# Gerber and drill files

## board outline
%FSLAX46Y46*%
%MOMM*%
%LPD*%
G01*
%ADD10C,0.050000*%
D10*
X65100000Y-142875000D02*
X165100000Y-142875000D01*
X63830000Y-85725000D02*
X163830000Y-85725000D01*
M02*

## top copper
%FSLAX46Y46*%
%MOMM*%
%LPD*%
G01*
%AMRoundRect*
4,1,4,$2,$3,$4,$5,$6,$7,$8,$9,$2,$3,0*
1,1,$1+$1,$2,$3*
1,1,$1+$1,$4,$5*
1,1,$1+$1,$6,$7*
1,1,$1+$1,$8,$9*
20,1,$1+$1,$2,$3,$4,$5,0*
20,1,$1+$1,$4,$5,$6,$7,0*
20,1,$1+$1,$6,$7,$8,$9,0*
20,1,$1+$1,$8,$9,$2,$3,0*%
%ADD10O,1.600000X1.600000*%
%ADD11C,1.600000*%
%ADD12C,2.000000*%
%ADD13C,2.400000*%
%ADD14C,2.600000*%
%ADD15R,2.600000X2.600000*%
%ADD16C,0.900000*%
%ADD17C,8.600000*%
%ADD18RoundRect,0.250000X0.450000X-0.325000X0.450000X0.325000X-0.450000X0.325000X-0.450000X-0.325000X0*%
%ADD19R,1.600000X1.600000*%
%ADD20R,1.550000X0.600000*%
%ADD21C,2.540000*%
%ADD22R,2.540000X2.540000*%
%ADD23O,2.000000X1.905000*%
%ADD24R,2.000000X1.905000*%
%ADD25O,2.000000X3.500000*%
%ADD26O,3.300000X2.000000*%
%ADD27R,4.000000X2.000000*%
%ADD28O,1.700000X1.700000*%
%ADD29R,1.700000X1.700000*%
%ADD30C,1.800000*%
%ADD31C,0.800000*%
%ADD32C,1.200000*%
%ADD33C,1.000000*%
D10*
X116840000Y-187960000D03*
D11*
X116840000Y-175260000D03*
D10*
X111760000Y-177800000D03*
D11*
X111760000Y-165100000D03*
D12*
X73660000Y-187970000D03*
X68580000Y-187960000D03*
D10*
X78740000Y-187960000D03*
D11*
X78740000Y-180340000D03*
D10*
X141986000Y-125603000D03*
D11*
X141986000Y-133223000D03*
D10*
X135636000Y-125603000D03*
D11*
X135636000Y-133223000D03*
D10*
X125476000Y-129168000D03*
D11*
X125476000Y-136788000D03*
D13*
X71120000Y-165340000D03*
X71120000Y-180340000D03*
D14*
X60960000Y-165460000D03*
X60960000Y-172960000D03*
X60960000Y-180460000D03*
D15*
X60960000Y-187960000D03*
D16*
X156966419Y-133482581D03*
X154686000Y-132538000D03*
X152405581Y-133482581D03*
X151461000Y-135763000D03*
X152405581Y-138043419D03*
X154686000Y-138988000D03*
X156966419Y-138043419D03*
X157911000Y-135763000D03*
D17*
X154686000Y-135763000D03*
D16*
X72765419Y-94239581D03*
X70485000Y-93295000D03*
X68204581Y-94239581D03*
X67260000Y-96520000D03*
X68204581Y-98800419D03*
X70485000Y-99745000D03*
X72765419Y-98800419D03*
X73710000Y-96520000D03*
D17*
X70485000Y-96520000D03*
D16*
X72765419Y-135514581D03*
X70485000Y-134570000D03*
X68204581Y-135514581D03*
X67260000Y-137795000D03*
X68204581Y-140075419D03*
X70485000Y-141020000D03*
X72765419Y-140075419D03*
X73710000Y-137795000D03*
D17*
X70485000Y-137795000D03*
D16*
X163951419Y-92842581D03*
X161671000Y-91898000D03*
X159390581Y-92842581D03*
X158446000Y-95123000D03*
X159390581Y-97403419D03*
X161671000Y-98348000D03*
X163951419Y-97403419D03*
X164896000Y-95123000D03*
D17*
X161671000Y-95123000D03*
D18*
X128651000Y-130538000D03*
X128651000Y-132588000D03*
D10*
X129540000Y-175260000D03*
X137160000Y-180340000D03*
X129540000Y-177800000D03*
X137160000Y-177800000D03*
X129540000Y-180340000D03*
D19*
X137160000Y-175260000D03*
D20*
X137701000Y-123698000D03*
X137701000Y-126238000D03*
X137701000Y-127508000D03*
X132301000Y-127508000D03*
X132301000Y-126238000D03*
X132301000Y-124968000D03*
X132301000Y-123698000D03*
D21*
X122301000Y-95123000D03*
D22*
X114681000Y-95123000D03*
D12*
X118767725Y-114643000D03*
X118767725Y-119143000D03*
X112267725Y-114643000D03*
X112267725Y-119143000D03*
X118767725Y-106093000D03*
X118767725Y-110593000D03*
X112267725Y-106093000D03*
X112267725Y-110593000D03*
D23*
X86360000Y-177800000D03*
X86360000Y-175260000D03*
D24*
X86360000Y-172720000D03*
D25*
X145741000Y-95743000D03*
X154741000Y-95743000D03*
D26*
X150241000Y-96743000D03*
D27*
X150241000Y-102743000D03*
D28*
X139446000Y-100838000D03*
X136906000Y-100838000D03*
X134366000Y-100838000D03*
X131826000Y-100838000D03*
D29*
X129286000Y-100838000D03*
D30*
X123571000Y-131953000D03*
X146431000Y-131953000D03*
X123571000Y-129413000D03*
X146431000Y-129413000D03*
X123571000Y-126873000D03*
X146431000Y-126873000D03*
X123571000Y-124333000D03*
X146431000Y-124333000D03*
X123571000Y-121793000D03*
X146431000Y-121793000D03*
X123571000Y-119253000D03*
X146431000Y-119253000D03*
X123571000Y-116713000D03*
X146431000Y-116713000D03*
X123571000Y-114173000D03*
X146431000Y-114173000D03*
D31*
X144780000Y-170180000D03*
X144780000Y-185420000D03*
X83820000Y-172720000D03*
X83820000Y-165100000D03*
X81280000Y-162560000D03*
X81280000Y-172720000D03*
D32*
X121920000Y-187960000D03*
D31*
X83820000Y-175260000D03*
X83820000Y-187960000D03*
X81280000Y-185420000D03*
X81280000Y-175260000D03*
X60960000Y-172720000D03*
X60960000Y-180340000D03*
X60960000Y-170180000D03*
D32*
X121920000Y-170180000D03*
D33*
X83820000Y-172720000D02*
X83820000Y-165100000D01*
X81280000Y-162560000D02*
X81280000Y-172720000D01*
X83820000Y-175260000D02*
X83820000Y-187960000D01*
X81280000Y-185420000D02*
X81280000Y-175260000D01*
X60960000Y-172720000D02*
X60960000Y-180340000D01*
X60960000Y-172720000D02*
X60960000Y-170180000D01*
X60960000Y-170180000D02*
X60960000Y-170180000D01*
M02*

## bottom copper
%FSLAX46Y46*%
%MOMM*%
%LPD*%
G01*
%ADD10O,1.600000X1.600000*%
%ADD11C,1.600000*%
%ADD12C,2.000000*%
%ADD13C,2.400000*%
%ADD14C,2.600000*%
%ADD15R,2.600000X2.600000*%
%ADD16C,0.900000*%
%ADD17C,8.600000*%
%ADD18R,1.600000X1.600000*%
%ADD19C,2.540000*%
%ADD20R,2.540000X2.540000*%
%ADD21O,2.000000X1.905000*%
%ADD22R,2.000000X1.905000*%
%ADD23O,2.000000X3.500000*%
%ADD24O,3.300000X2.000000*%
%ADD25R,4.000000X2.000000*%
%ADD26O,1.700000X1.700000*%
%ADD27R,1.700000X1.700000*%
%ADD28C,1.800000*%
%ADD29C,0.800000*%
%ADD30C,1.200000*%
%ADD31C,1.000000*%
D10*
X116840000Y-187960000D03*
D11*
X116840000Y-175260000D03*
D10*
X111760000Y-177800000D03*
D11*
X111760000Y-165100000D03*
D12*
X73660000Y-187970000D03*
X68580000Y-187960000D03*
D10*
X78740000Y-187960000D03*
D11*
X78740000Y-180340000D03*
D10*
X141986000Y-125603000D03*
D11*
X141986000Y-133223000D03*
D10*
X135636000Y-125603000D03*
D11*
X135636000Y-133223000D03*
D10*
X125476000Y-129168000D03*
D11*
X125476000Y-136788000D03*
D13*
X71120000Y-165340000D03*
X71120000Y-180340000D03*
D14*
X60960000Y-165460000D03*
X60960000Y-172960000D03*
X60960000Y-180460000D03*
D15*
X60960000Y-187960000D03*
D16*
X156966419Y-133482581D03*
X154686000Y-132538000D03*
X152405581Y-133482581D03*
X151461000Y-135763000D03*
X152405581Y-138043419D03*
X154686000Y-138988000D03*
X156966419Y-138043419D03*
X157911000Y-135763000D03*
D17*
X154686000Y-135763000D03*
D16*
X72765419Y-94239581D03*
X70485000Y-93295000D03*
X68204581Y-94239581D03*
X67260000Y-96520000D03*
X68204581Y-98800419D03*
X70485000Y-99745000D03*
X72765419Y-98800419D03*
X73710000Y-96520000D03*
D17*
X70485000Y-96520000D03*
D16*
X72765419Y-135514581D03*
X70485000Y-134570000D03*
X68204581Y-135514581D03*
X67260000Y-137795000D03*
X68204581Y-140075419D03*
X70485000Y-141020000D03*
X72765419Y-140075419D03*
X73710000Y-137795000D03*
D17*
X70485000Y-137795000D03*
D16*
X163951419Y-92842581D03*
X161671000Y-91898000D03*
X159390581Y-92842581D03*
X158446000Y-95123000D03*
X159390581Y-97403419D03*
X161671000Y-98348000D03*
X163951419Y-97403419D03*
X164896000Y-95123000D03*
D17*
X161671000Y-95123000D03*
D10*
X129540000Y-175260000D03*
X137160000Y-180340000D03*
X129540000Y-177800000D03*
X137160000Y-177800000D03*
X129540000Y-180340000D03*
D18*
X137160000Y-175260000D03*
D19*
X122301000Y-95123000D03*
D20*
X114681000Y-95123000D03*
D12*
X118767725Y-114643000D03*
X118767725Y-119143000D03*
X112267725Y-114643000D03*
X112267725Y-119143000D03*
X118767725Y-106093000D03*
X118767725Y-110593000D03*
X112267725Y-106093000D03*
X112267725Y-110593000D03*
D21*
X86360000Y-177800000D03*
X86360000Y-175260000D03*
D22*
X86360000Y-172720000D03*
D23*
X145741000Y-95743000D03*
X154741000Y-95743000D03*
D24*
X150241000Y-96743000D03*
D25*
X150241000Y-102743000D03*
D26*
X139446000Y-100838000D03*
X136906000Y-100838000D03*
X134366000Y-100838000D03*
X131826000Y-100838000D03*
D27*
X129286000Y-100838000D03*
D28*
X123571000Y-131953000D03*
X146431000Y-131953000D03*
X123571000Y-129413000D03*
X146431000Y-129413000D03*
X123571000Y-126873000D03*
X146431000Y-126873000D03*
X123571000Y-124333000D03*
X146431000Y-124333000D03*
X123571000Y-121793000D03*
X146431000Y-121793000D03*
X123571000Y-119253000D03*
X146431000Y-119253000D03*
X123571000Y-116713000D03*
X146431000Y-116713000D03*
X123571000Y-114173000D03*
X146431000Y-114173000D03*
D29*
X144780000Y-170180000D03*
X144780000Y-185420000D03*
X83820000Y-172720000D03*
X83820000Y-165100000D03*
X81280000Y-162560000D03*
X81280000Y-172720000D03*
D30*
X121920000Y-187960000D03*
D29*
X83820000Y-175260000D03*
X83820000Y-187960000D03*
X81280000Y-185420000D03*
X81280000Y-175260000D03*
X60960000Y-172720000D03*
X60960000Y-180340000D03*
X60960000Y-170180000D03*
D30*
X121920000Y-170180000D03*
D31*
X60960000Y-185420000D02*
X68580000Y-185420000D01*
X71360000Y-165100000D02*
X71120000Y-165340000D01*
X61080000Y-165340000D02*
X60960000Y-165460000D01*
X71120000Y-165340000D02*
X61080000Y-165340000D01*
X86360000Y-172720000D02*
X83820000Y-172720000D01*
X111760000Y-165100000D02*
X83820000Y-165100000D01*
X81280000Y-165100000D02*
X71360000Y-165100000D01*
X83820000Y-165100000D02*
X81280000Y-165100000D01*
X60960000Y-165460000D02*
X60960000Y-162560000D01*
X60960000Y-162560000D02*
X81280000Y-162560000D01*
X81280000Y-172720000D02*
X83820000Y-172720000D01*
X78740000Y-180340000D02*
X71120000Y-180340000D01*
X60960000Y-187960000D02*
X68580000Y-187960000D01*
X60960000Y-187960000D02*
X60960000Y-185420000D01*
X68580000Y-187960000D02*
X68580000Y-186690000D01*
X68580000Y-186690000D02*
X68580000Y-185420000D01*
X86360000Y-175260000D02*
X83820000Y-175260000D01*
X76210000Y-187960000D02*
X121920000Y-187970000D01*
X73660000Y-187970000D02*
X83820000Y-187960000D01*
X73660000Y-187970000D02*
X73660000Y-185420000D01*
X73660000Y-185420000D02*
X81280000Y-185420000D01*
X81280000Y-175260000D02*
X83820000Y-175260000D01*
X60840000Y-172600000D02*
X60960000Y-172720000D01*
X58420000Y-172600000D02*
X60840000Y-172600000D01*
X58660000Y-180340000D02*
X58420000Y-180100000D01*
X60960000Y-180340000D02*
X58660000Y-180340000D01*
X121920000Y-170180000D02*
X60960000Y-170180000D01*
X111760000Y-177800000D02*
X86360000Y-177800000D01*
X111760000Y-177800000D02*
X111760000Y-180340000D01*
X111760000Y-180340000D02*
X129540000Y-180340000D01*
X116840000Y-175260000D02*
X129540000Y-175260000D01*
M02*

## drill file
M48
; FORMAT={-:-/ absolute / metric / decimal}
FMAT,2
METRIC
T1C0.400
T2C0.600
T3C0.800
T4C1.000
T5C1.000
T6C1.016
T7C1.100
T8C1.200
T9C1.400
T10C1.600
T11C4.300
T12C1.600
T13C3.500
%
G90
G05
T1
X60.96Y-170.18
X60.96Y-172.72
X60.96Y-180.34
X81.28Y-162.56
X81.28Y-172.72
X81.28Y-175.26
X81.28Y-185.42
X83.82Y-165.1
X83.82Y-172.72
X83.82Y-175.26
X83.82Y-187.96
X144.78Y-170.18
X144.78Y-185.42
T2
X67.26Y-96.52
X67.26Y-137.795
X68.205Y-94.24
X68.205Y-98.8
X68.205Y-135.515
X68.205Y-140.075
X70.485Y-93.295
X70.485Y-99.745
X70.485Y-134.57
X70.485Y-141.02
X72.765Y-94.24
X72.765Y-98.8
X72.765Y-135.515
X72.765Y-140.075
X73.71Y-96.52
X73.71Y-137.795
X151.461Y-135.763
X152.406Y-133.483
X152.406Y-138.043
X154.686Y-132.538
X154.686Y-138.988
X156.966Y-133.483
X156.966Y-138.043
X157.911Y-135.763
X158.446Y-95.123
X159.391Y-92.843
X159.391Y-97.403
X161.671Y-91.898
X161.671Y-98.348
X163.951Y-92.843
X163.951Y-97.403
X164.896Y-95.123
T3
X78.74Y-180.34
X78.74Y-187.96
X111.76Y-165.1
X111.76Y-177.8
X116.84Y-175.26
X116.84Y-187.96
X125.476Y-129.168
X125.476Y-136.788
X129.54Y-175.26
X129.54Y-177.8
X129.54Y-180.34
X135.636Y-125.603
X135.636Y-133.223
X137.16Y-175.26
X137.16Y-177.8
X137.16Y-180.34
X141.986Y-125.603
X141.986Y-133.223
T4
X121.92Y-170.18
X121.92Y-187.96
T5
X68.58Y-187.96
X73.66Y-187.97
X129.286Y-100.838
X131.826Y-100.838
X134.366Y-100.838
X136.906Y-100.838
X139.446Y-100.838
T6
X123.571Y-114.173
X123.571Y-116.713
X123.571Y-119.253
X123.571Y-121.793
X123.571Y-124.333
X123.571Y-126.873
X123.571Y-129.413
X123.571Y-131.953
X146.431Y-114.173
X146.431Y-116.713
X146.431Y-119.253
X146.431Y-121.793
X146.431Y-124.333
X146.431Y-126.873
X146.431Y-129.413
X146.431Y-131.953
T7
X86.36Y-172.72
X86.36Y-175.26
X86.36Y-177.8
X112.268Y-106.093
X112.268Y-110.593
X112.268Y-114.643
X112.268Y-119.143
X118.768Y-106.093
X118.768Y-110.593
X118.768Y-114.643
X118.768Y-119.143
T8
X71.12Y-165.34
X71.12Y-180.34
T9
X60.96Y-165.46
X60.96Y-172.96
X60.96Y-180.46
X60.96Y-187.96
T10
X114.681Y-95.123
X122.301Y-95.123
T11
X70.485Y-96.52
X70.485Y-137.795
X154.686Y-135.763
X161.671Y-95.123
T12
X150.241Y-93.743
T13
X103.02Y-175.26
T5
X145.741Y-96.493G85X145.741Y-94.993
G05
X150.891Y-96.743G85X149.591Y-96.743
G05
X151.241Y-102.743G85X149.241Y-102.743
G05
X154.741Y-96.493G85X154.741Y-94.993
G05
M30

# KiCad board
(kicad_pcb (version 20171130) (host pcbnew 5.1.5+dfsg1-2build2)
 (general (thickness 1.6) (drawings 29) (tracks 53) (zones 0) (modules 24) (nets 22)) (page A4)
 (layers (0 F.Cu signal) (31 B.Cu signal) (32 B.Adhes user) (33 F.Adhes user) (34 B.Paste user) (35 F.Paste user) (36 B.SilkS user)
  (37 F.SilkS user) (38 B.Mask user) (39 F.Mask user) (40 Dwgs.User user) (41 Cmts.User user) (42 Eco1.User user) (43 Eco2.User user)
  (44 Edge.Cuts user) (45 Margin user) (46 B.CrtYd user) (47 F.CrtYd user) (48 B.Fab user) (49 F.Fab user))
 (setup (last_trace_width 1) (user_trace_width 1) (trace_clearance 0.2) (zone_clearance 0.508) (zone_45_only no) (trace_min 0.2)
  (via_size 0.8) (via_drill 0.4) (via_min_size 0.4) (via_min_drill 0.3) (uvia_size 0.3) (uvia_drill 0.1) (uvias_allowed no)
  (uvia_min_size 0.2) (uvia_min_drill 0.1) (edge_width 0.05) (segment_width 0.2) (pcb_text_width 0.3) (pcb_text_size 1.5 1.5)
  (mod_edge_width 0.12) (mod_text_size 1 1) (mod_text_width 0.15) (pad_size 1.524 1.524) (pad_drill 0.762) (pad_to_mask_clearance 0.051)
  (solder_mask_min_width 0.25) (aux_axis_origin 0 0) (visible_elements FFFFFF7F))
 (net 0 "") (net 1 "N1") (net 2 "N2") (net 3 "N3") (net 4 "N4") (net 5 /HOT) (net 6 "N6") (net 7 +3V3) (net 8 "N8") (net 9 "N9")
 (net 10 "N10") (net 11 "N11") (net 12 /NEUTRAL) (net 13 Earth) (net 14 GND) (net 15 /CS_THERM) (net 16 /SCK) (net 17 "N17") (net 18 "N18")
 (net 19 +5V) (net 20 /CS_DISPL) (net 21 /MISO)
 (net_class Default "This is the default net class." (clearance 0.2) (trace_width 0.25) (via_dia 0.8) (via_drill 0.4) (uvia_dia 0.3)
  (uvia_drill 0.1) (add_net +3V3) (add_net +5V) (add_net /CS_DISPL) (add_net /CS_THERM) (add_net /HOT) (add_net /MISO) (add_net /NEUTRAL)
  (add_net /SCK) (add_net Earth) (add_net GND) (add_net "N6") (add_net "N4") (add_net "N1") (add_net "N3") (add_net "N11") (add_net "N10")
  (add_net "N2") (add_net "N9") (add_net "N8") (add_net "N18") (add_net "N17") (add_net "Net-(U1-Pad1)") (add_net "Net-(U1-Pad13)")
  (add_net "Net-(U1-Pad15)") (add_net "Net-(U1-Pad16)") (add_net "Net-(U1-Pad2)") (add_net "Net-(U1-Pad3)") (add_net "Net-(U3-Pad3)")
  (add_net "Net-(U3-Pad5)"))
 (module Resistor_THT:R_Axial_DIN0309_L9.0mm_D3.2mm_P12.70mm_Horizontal (layer F.Cu) (at 116.84 175.26 270)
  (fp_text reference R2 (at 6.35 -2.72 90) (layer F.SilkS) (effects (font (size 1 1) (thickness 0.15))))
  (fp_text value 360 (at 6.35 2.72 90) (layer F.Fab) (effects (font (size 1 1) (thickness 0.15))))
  (pad 2 thru_hole oval (at 12.7 0 270) (size 1.6 1.6) (drill 0.8) (layers *.Cu *.Mask) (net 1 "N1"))
  (pad 1 thru_hole circle (at 0 0 270) (size 1.6 1.6) (drill 0.8) (layers *.Cu *.Mask) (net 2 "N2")))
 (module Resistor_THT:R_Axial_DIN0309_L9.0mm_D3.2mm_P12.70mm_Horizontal (layer F.Cu) (at 111.76 165.1 270)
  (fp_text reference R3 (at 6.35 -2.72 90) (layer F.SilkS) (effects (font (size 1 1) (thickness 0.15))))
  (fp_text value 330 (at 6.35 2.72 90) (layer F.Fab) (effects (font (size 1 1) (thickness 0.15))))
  (pad 2 thru_hole oval (at 12.7 0 270) (size 1.6 1.6) (drill 0.8) (layers *.Cu *.Mask) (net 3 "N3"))
  (pad 1 thru_hole circle (at 0 0 270) (size 1.6 1.6) (drill 0.8) (layers *.Cu *.Mask) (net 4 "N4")))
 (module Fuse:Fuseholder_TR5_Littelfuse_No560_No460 (layer F.Cu) (at 68.58 187.96)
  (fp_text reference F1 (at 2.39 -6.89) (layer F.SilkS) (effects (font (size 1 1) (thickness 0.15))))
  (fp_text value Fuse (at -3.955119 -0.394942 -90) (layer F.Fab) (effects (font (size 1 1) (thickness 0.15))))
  (pad 2 thru_hole circle (at 5.08 0.01) (size 2 2) (drill 1) (layers *.Cu *.Mask) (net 1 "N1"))
  (pad 1 thru_hole circle (at 0 0) (size 2 2) (drill 1) (layers *.Cu *.Mask) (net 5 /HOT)))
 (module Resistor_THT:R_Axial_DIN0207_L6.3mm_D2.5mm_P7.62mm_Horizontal (layer F.Cu) (at 78.74 180.34 270)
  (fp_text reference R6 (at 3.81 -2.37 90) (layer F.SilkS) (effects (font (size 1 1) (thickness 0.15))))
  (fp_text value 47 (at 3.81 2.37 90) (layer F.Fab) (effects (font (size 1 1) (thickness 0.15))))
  (pad 2 thru_hole oval (at 7.62 0 270) (size 1.6 1.6) (drill 0.8) (layers *.Cu *.Mask) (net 1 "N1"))
  (pad 1 thru_hole circle (at 0 0 270) (size 1.6 1.6) (drill 0.8) (layers *.Cu *.Mask) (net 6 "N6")))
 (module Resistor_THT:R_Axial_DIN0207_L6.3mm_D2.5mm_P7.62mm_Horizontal (layer F.Cu) (at 141.986 133.223 90)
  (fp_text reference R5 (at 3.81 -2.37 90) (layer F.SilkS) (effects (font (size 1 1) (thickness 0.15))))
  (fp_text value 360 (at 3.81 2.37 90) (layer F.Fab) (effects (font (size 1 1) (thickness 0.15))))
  (pad 2 thru_hole oval (at 7.62 0 90) (size 1.6 1.6) (drill 0.8) (layers *.Cu *.Mask) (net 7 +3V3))
  (pad 1 thru_hole circle (at 0 0 90) (size 1.6 1.6) (drill 0.8) (layers *.Cu *.Mask) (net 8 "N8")))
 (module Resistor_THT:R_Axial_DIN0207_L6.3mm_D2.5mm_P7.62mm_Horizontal (layer F.Cu) (at 135.636 133.223 90)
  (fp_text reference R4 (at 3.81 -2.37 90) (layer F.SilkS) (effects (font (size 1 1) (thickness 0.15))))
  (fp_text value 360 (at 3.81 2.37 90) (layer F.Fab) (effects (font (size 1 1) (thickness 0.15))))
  (pad 2 thru_hole oval (at 7.62 0 90) (size 1.6 1.6) (drill 0.8) (layers *.Cu *.Mask) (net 7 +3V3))
  (pad 1 thru_hole circle (at 0 0 90) (size 1.6 1.6) (drill 0.8) (layers *.Cu *.Mask) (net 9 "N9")))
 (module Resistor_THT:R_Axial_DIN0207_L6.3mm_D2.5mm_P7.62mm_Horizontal (layer F.Cu) (at 125.476 136.788 90)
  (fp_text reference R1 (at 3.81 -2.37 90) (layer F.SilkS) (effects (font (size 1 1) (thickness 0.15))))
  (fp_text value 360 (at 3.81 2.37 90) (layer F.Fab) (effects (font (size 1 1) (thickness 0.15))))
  (pad 2 thru_hole oval (at 7.62 0 90) (size 1.6 1.6) (drill 0.8) (layers *.Cu *.Mask) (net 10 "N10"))
  (pad 1 thru_hole circle (at 0 0 90) (size 1.6 1.6) (drill 0.8) (layers *.Cu *.Mask) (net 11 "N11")))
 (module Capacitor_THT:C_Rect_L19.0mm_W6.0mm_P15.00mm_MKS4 (layer F.Cu) (at 71.12 180.34 90)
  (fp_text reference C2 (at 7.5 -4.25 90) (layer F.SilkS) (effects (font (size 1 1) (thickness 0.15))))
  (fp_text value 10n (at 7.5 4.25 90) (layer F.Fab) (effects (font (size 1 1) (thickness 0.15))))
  (pad 2 thru_hole circle (at 15 0 90) (size 2.4 2.4) (drill 1.2) (layers *.Cu *.Mask) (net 4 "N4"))
  (pad 1 thru_hole circle (at 0 0 90) (size 2.4 2.4) (drill 1.2) (layers *.Cu *.Mask) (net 6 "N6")))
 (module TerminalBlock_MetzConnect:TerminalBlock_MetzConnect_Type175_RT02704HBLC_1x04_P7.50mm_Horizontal (layer F.Cu) (at 60.96 187.96 90)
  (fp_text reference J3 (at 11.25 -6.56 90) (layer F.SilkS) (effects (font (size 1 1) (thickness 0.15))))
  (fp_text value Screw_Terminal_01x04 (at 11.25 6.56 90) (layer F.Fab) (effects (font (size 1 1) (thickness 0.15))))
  (pad 4 thru_hole circle (at 22.5 0 90) (size 2.6 2.6) (drill 1.4) (layers *.Cu *.Mask) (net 4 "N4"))
  (pad 3 thru_hole circle (at 15 0 90) (size 2.6 2.6) (drill 1.4) (layers *.Cu *.Mask) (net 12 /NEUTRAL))
  (pad 2 thru_hole circle (at 7.5 0 90) (size 2.6 2.6) (drill 1.4) (layers *.Cu *.Mask) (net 12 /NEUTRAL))
  (pad 1 thru_hole rect (at 0 0 90) (size 2.6 2.6) (drill 1.4) (layers *.Cu *.Mask) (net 5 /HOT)))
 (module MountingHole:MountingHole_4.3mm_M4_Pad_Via (layer F.Cu) (at 154.686 135.763)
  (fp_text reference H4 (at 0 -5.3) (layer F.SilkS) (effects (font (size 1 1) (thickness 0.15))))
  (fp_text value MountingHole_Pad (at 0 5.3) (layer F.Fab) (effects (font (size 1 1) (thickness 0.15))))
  (pad 1 thru_hole circle (at 2.280419 -2.280419) (size 0.9 0.9) (drill 0.6) (layers *.Cu *.Mask) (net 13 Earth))
  (pad 1 thru_hole circle (at 0 -3.225) (size 0.9 0.9) (drill 0.6) (layers *.Cu *.Mask) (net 13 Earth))
  (pad 1 thru_hole circle (at -2.280419 -2.280419) (size 0.9 0.9) (drill 0.6) (layers *.Cu *.Mask) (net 13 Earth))
  (pad 1 thru_hole circle (at -3.225 0) (size 0.9 0.9) (drill 0.6) (layers *.Cu *.Mask) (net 13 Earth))
  (pad 1 thru_hole circle (at -2.280419 2.280419) (size 0.9 0.9) (drill 0.6) (layers *.Cu *.Mask) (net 13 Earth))
  (pad 1 thru_hole circle (at 0 3.225) (size 0.9 0.9) (drill 0.6) (layers *.Cu *.Mask) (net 13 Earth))
  (pad 1 thru_hole circle (at 2.280419 2.280419) (size 0.9 0.9) (drill 0.6) (layers *.Cu *.Mask) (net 13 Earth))
  (pad 1 thru_hole circle (at 3.225 0) (size 0.9 0.9) (drill 0.6) (layers *.Cu *.Mask) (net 13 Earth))
  (pad 1 thru_hole circle (at 0 0) (size 8.6 8.6) (drill 4.3) (layers *.Cu *.Mask) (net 13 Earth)))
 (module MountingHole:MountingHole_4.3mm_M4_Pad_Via (layer F.Cu) (at 70.485 96.52)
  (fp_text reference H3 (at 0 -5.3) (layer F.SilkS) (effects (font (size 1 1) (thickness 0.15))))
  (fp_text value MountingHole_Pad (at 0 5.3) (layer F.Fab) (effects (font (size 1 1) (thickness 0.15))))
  (pad 1 thru_hole circle (at 2.280419 -2.280419) (size 0.9 0.9) (drill 0.6) (layers *.Cu *.Mask) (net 13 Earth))
  (pad 1 thru_hole circle (at 0 -3.225) (size 0.9 0.9) (drill 0.6) (layers *.Cu *.Mask) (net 13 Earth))
  (pad 1 thru_hole circle (at -2.280419 -2.280419) (size 0.9 0.9) (drill 0.6) (layers *.Cu *.Mask) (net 13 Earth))
  (pad 1 thru_hole circle (at -3.225 0) (size 0.9 0.9) (drill 0.6) (layers *.Cu *.Mask) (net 13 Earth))
  (pad 1 thru_hole circle (at -2.280419 2.280419) (size 0.9 0.9) (drill 0.6) (layers *.Cu *.Mask) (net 13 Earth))
  (pad 1 thru_hole circle (at 0 3.225) (size 0.9 0.9) (drill 0.6) (layers *.Cu *.Mask) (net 13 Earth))
  (pad 1 thru_hole circle (at 2.280419 2.280419) (size 0.9 0.9) (drill 0.6) (layers *.Cu *.Mask) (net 13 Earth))
  (pad 1 thru_hole circle (at 3.225 0) (size 0.9 0.9) (drill 0.6) (layers *.Cu *.Mask) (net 13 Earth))
  (pad 1 thru_hole circle (at 0 0) (size 8.6 8.6) (drill 4.3) (layers *.Cu *.Mask) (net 13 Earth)))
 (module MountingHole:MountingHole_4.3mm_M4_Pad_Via (layer F.Cu) (at 70.485 137.795)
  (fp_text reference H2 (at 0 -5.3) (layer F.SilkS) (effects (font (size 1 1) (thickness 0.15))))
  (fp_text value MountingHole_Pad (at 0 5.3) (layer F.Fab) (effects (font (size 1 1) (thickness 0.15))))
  (pad 1 thru_hole circle (at 2.280419 -2.280419) (size 0.9 0.9) (drill 0.6) (layers *.Cu *.Mask) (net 13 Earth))
  (pad 1 thru_hole circle (at 0 -3.225) (size 0.9 0.9) (drill 0.6) (layers *.Cu *.Mask) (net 13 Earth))
  (pad 1 thru_hole circle (at -2.280419 -2.280419) (size 0.9 0.9) (drill 0.6) (layers *.Cu *.Mask) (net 13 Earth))
  (pad 1 thru_hole circle (at -3.225 0) (size 0.9 0.9) (drill 0.6) (layers *.Cu *.Mask) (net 13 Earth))
  (pad 1 thru_hole circle (at -2.280419 2.280419) (size 0.9 0.9) (drill 0.6) (layers *.Cu *.Mask) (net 13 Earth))
  (pad 1 thru_hole circle (at 0 3.225) (size 0.9 0.9) (drill 0.6) (layers *.Cu *.Mask) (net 13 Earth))
  (pad 1 thru_hole circle (at 2.280419 2.280419) (size 0.9 0.9) (drill 0.6) (layers *.Cu *.Mask) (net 13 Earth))
  (pad 1 thru_hole circle (at 3.225 0) (size 0.9 0.9) (drill 0.6) (layers *.Cu *.Mask) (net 13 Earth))
  (pad 1 thru_hole circle (at 0 0) (size 8.6 8.6) (drill 4.3) (layers *.Cu *.Mask) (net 13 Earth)))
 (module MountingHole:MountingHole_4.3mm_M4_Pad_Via (layer F.Cu) (at 161.671 95.123)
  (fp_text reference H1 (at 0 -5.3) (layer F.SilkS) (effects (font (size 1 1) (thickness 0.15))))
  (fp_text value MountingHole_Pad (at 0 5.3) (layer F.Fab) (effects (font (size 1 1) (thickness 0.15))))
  (pad 1 thru_hole circle (at 2.280419 -2.280419) (size 0.9 0.9) (drill 0.6) (layers *.Cu *.Mask) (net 13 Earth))
  (pad 1 thru_hole circle (at 0 -3.225) (size 0.9 0.9) (drill 0.6) (layers *.Cu *.Mask) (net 13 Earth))
  (pad 1 thru_hole circle (at -2.280419 -2.280419) (size 0.9 0.9) (drill 0.6) (layers *.Cu *.Mask) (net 13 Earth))
  (pad 1 thru_hole circle (at -3.225 0) (size 0.9 0.9) (drill 0.6) (layers *.Cu *.Mask) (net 13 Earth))
  (pad 1 thru_hole circle (at -2.280419 2.280419) (size 0.9 0.9) (drill 0.6) (layers *.Cu *.Mask) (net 13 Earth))
  (pad 1 thru_hole circle (at 0 3.225) (size 0.9 0.9) (drill 0.6) (layers *.Cu *.Mask) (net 13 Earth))
  (pad 1 thru_hole circle (at 2.280419 2.280419) (size 0.9 0.9) (drill 0.6) (layers *.Cu *.Mask) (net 13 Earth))
  (pad 1 thru_hole circle (at 3.225 0) (size 0.9 0.9) (drill 0.6) (layers *.Cu *.Mask) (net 13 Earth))
  (pad 1 thru_hole circle (at 0 0) (size 8.6 8.6) (drill 4.3) (layers *.Cu *.Mask) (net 13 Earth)))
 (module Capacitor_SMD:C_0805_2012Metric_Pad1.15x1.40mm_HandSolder (layer F.Cu) (at 128.651 131.563 90)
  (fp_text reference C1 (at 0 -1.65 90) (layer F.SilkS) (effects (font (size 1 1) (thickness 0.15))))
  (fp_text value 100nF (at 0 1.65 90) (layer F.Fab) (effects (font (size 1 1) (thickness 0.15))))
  (pad 2 smd roundrect (at 1.025 0 90) (size 1.15 1.4) (layers F.Cu F.Paste F.Mask) (roundrect_rratio 0.217391) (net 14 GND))
  (pad 1 smd roundrect (at -1.025 0 90) (size 1.15 1.4) (layers F.Cu F.Paste F.Mask) (roundrect_rratio 0.217391) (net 7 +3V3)))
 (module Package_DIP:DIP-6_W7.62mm (layer B.Cu) (at 137.16 175.26 180)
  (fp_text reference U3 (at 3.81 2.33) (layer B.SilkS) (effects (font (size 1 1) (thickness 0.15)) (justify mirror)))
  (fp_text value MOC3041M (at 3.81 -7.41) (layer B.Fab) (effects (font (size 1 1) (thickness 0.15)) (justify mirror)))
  (pad 6 thru_hole oval (at 7.62 0 180) (size 1.6 1.6) (drill 0.8) (layers *.Cu *.Mask) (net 2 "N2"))
  (pad 3 thru_hole oval (at 0 -5.08 180) (size 1.6 1.6) (drill 0.8) (layers *.Cu *.Mask))
  (pad 5 thru_hole oval (at 7.62 -2.54 180) (size 1.6 1.6) (drill 0.8) (layers *.Cu *.Mask))
  (pad 2 thru_hole oval (at 0 -2.54 180) (size 1.6 1.6) (drill 0.8) (layers *.Cu *.Mask) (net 14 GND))
  (pad 4 thru_hole oval (at 7.62 -5.08 180) (size 1.6 1.6) (drill 0.8) (layers *.Cu *.Mask) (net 3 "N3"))
  (pad 1 thru_hole rect (at 0 0 180) (size 1.6 1.6) (drill 0.8) (layers *.Cu *.Mask) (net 11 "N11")))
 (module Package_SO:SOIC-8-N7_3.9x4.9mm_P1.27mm (layer F.Cu) (at 135.001 125.603)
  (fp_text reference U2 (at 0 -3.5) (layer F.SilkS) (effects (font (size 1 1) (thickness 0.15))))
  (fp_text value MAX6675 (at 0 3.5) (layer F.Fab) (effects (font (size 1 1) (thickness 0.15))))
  (pad 8 smd rect (at 2.7 -1.905) (size 1.55 0.6) (layers F.Cu F.Paste F.Mask))
  (pad 6 smd rect (at 2.7 0.635) (size 1.55 0.6) (layers F.Cu F.Paste F.Mask) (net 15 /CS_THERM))
  (pad 5 smd rect (at 2.7 1.905) (size 1.55 0.6) (layers F.Cu F.Paste F.Mask) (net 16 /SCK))
  (pad 4 smd rect (at -2.7 1.905) (size 1.55 0.6) (layers F.Cu F.Paste F.Mask) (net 7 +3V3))
  (pad 3 smd rect (at -2.7 0.635) (size 1.55 0.6) (layers F.Cu F.Paste F.Mask) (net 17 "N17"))
  (pad 2 smd rect (at -2.7 -0.635) (size 1.55 0.6) (layers F.Cu F.Paste F.Mask) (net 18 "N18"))
  (pad 1 smd rect (at -2.7 -1.905) (size 1.55 0.6) (layers F.Cu F.Paste F.Mask) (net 14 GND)))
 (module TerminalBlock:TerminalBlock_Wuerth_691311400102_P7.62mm (layer F.Cu) (at 114.681 95.123)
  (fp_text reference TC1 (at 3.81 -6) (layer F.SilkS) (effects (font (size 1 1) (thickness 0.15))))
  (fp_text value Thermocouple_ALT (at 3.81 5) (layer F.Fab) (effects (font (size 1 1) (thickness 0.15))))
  (pad 2 thru_hole circle (at 7.62 0) (size 2.54 2.54) (drill 1.6) (layers *.Cu *.Mask) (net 17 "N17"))
  (pad 1 thru_hole rect (at 0 0) (size 2.54 2.54) (drill 1.6) (layers *.Cu *.Mask) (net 18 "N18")))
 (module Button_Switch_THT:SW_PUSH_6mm (layer F.Cu) (at 112.267725 114.643)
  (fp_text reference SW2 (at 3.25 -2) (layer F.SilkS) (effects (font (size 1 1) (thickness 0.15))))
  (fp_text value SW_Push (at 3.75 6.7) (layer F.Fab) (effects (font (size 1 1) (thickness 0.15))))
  (pad 1 thru_hole circle (at 6.5 0 90) (size 2 2) (drill 1.1) (layers *.Cu *.Mask) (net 8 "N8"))
  (pad 2 thru_hole circle (at 6.5 4.5 90) (size 2 2) (drill 1.1) (layers *.Cu *.Mask) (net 14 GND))
  (pad 1 thru_hole circle (at 0 0 90) (size 2 2) (drill 1.1) (layers *.Cu *.Mask) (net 8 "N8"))
  (pad 2 thru_hole circle (at 0 4.5 90) (size 2 2) (drill 1.1) (layers *.Cu *.Mask) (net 14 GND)))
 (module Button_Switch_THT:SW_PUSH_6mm (layer F.Cu) (at 112.267725 106.093)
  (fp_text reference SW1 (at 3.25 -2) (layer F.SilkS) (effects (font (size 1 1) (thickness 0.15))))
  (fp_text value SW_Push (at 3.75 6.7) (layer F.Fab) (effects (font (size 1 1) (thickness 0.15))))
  (pad 1 thru_hole circle (at 6.5 0 90) (size 2 2) (drill 1.1) (layers *.Cu *.Mask) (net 9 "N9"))
  (pad 2 thru_hole circle (at 6.5 4.5 90) (size 2 2) (drill 1.1) (layers *.Cu *.Mask) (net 14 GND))
  (pad 1 thru_hole circle (at 0 0 90) (size 2 2) (drill 1.1) (layers *.Cu *.Mask) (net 9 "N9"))
  (pad 2 thru_hole circle (at 0 4.5 90) (size 2 2) (drill 1.1) (layers *.Cu *.Mask) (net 14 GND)))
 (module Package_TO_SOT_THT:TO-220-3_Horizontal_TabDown (layer F.Cu) (at 86.36 172.72 270)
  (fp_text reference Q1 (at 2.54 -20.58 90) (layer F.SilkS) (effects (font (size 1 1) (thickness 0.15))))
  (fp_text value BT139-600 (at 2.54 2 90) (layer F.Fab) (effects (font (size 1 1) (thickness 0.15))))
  (pad 3 thru_hole oval (at 5.08 0 270) (size 1.905 2) (drill 1.1) (layers *.Cu *.Mask) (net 3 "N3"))
  (pad 2 thru_hole oval (at 2.54 0 270) (size 1.905 2) (drill 1.1) (layers *.Cu *.Mask) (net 1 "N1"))
  (pad 1 thru_hole rect (at 0 0 270) (size 1.905 2) (drill 1.1) (layers *.Cu *.Mask) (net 4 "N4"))
  (pad "" np_thru_hole oval (at 2.54 -16.66 270) (size 3.5 3.5) (drill 3.5) (layers *.Cu *.Mask)))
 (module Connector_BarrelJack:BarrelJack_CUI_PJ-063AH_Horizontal (layer F.Cu) (at 150.241 102.743 180)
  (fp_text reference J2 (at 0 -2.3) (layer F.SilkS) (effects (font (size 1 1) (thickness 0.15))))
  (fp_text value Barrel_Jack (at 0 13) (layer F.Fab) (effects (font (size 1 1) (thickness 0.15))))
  (pad "" np_thru_hole circle (at 0 9 180) (size 1.6 1.6) (drill 1.6) (layers *.Cu *.Mask))
  (pad MP thru_hole oval (at 4.5 7 180) (size 2 3.5) (drill oval 1 2.5) (layers *.Cu *.Mask))
  (pad MP thru_hole oval (at -4.5 7 180) (size 2 3.5) (drill oval 1 2.5) (layers *.Cu *.Mask))
  (pad 2 thru_hole oval (at 0 6 180) (size 3.3 2) (drill oval 2.3 1) (layers *.Cu *.Mask) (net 14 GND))
  (pad 1 thru_hole rect (at 0 0 180) (size 4 2) (drill oval 3 1) (layers *.Cu *.Mask) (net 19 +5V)))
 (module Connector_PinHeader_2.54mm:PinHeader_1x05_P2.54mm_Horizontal (layer F.Cu) (at 129.286 100.838 90)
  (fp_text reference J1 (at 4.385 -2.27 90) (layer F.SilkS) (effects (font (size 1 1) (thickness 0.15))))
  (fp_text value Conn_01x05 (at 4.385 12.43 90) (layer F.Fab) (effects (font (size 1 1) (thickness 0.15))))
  (pad 5 thru_hole oval (at 0 10.16 90) (size 1.7 1.7) (drill 1) (layers *.Cu *.Mask) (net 14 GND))
  (pad 4 thru_hole oval (at 0 7.62 90) (size 1.7 1.7) (drill 1) (layers *.Cu *.Mask) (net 19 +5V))
  (pad 3 thru_hole oval (at 0 5.08 90) (size 1.7 1.7) (drill 1) (layers *.Cu *.Mask) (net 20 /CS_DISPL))
  (pad 2 thru_hole oval (at 0 2.54 90) (size 1.7 1.7) (drill 1) (layers *.Cu *.Mask) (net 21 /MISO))
  (pad 1 thru_hole rect (at 0 0 90) (size 1.7 1.7) (drill 1) (layers *.Cu *.Mask) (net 16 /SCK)))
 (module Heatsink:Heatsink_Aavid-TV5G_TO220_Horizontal (layer F.Cu) (at 87.884 110.8075)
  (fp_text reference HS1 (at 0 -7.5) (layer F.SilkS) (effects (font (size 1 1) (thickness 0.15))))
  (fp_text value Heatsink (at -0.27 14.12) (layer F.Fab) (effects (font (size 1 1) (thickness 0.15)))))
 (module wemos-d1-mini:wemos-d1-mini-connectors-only (layer F.Cu) (at 135.001 123.063 270)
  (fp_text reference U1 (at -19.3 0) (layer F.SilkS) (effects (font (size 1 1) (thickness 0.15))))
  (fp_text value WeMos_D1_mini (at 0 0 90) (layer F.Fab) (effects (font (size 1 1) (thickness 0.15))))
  (pad 16 thru_hole circle (at 8.89 11.43 270) (size 1.8 1.8) (drill 1.016) (layers *.Cu *.Mask))
  (pad 1 thru_hole circle (at 8.89 -11.43 270) (size 1.8 1.8) (drill 1.016) (layers *.Cu *.Mask))
  (pad 15 thru_hole circle (at 6.35 11.43 270) (size 1.8 1.8) (drill 1.016) (layers *.Cu *.Mask))
  (pad 2 thru_hole circle (at 6.35 -11.43 270) (size 1.8 1.8) (drill 1.016) (layers *.Cu *.Mask))
  (pad 14 thru_hole circle (at 3.81 11.43 270) (size 1.8 1.8) (drill 1.016) (layers *.Cu *.Mask) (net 10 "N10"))
  (pad 3 thru_hole circle (at 3.81 -11.43 270) (size 1.8 1.8) (drill 1.016) (layers *.Cu *.Mask))
  (pad 13 thru_hole circle (at 1.27 11.43 270) (size 1.8 1.8) (drill 1.016) (layers *.Cu *.Mask))
  (pad 4 thru_hole circle (at 1.27 -11.43 270) (size 1.8 1.8) (drill 1.016) (layers *.Cu *.Mask) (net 16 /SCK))
  (pad 12 thru_hole circle (at -1.27 11.43 270) (size 1.8 1.8) (drill 1.016) (layers *.Cu *.Mask) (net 8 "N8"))
  (pad 5 thru_hole circle (at -1.27 -11.43 270) (size 1.8 1.8) (drill 1.016) (layers *.Cu *.Mask) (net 21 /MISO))
  (pad 11 thru_hole circle (at -3.81 11.43 270) (size 1.8 1.8) (drill 1.016) (layers *.Cu *.Mask) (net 9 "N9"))
  (pad 6 thru_hole circle (at -3.81 -11.43 270) (size 1.8 1.8) (drill 1.016) (layers *.Cu *.Mask) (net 15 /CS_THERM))
  (pad 10 thru_hole circle (at -6.35 11.43 270) (size 1.8 1.8) (drill 1.016) (layers *.Cu *.Mask) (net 14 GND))
  (pad 7 thru_hole circle (at -6.35 -11.43 270) (size 1.8 1.8) (drill 1.016) (layers *.Cu *.Mask) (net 20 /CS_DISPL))
  (pad 9 thru_hole circle (at -8.89 11.43 270) (size 1.8 1.8) (drill 1.016) (layers *.Cu *.Mask) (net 19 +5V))
  (pad 8 thru_hole circle (at -8.89 -11.43 270) (size 1.8 1.8) (drill 1.016) (layers *.Cu *.Mask) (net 7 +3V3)))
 (gr_line (start 65.1 142.875) (end 165.1 142.875) (layer Edge.Cuts) (width 0.05))
 (gr_line (start 63.83 85.725) (end 163.83 85.725) (layer Edge.Cuts) (width 0.05))
 (via (at 144.78 170.18) (size 0.8) (drill 0.4) (layers F.Cu B.Cu) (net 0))
 (via (at 144.78 185.42) (size 0.8) (drill 0.4) (layers F.Cu B.Cu) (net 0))
 (segment (start 60.96 185.42) (end 68.58 185.42) (width 1) (layer B.Cu) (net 5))
 (segment (start 71.36 165.1) (end 71.12 165.34) (width 1) (layer B.Cu) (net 4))
 (segment (start 61.08 165.34) (end 60.96 165.46) (width 1) (layer B.Cu) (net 4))
 (segment (start 71.12 165.34) (end 61.08 165.34) (width 1) (layer B.Cu) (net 4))
 (via (at 83.82 172.72) (size 0.8) (drill 0.4) (layers F.Cu B.Cu) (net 4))
 (segment (start 86.36 172.72) (end 83.82 172.72) (width 1) (layer B.Cu) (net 4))
 (via (at 83.82 165.1) (size 0.8) (drill 0.4) (layers F.Cu B.Cu) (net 4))
 (segment (start 83.82 172.72) (end 83.82 165.1) (width 1) (layer F.Cu) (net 4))
 (segment (start 111.76 165.1) (end 83.82 165.1) (width 1) (layer B.Cu) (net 4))
 (segment (start 81.28 165.1) (end 71.36 165.1) (width 1) (layer B.Cu) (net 4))
 (segment (start 83.82 165.1) (end 81.28 165.1) (width 1) (layer B.Cu) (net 4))
 (segment (start 60.96 165.46) (end 60.96 162.56) (width 1) (layer B.Cu) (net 4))
 (via (at 81.28 162.56) (size 0.8) (drill 0.4) (layers F.Cu B.Cu) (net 4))
 (segment (start 60.96 162.56) (end 81.28 162.56) (width 1) (layer B.Cu) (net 4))
 (via (at 81.28 172.72) (size 0.8) (drill 0.4) (layers F.Cu B.Cu) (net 4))
 (segment (start 81.28 162.56) (end 81.28 172.72) (width 1) (layer F.Cu) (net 4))
 (segment (start 81.28 172.72) (end 83.82 172.72) (width 1) (layer B.Cu) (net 4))
 (segment (start 78.74 180.34) (end 71.12 180.34) (width 1) (layer B.Cu) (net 6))
 (segment (start 60.96 187.96) (end 68.58 187.96) (width 1) (layer B.Cu) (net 5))
 (segment (start 60.96 187.96) (end 60.96 185.42) (width 1) (layer B.Cu) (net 5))
 (segment (start 68.58 187.96) (end 68.58 186.69) (width 1) (layer B.Cu) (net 5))
 (segment (start 68.58 186.69) (end 68.58 185.42) (width 1) (layer B.Cu) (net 5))
 (via (at 121.92 187.96) (size 1.2) (drill 1) (layers F.Cu B.Cu) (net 1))
 (via (at 83.82 175.26) (size 0.8) (drill 0.4) (layers F.Cu B.Cu) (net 1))
 (segment (start 86.36 175.26) (end 83.82 175.26) (width 1) (layer B.Cu) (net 1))
 (via (at 83.82 187.96) (size 0.8) (drill 0.4) (layers F.Cu B.Cu) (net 1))
 (segment (start 83.82 175.26) (end 83.82 187.96) (width 1) (layer F.Cu) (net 1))
 (segment (start 76.21 187.96) (end 121.92 187.97) (width 1) (layer B.Cu) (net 1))
 (segment (start 73.66 187.97) (end 83.82 187.96) (width 1) (layer B.Cu) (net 1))
 (segment (start 73.66 187.97) (end 73.66 185.42) (width 1) (layer B.Cu) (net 1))
 (via (at 81.28 185.42) (size 0.8) (drill 0.4) (layers F.Cu B.Cu) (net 1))
 (segment (start 73.66 185.42) (end 81.28 185.42) (width 1) (layer B.Cu) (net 1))
 (via (at 81.28 175.26) (size 0.8) (drill 0.4) (layers F.Cu B.Cu) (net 1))
 (segment (start 81.28 185.42) (end 81.28 175.26) (width 1) (layer F.Cu) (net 1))
 (segment (start 81.28 175.26) (end 83.82 175.26) (width 1) (layer B.Cu) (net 1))
 (via (at 60.96 172.72) (size 0.8) (drill 0.4) (layers F.Cu B.Cu) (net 12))
 (segment (start 60.84 172.6) (end 60.96 172.72) (width 1) (layer B.Cu) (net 12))
 (segment (start 58.42 172.6) (end 60.84 172.6) (width 1) (layer B.Cu) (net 12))
 (via (at 60.96 180.34) (size 0.8) (drill 0.4) (layers F.Cu B.Cu) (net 12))
 (segment (start 60.96 172.72) (end 60.96 180.34) (width 1) (layer F.Cu) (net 12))
 (segment (start 58.66 180.34) (end 58.42 180.1) (width 1) (layer B.Cu) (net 12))
 (segment (start 60.96 180.34) (end 58.66 180.34) (width 1) (layer B.Cu) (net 12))
 (segment (start 60.96 172.72) (end 60.96 170.18) (width 1) (layer F.Cu) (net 12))
 (segment (start 60.96 170.18) (end 60.96 170.18) (width 1) (layer F.Cu) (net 12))
 (via (at 60.96 170.18) (size 0.8) (drill 0.4) (layers F.Cu B.Cu) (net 12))
 (segment (start 121.92 170.18) (end 60.96 170.18) (width 1) (layer B.Cu) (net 12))
 (via (at 121.92 170.18) (size 1.2) (drill 1) (layers F.Cu B.Cu) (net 12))
 (segment (start 111.76 177.8) (end 86.36 177.8) (width 1) (layer B.Cu) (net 3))
 (segment (start 111.76 177.8) (end 111.76 180.34) (width 1) (layer B.Cu) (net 3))
 (segment (start 111.76 180.34) (end 129.54 180.34) (width 1) (layer B.Cu) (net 3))
 (segment (start 116.84 175.26) (end 129.54 175.26) (width 1) (layer B.Cu) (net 2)))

